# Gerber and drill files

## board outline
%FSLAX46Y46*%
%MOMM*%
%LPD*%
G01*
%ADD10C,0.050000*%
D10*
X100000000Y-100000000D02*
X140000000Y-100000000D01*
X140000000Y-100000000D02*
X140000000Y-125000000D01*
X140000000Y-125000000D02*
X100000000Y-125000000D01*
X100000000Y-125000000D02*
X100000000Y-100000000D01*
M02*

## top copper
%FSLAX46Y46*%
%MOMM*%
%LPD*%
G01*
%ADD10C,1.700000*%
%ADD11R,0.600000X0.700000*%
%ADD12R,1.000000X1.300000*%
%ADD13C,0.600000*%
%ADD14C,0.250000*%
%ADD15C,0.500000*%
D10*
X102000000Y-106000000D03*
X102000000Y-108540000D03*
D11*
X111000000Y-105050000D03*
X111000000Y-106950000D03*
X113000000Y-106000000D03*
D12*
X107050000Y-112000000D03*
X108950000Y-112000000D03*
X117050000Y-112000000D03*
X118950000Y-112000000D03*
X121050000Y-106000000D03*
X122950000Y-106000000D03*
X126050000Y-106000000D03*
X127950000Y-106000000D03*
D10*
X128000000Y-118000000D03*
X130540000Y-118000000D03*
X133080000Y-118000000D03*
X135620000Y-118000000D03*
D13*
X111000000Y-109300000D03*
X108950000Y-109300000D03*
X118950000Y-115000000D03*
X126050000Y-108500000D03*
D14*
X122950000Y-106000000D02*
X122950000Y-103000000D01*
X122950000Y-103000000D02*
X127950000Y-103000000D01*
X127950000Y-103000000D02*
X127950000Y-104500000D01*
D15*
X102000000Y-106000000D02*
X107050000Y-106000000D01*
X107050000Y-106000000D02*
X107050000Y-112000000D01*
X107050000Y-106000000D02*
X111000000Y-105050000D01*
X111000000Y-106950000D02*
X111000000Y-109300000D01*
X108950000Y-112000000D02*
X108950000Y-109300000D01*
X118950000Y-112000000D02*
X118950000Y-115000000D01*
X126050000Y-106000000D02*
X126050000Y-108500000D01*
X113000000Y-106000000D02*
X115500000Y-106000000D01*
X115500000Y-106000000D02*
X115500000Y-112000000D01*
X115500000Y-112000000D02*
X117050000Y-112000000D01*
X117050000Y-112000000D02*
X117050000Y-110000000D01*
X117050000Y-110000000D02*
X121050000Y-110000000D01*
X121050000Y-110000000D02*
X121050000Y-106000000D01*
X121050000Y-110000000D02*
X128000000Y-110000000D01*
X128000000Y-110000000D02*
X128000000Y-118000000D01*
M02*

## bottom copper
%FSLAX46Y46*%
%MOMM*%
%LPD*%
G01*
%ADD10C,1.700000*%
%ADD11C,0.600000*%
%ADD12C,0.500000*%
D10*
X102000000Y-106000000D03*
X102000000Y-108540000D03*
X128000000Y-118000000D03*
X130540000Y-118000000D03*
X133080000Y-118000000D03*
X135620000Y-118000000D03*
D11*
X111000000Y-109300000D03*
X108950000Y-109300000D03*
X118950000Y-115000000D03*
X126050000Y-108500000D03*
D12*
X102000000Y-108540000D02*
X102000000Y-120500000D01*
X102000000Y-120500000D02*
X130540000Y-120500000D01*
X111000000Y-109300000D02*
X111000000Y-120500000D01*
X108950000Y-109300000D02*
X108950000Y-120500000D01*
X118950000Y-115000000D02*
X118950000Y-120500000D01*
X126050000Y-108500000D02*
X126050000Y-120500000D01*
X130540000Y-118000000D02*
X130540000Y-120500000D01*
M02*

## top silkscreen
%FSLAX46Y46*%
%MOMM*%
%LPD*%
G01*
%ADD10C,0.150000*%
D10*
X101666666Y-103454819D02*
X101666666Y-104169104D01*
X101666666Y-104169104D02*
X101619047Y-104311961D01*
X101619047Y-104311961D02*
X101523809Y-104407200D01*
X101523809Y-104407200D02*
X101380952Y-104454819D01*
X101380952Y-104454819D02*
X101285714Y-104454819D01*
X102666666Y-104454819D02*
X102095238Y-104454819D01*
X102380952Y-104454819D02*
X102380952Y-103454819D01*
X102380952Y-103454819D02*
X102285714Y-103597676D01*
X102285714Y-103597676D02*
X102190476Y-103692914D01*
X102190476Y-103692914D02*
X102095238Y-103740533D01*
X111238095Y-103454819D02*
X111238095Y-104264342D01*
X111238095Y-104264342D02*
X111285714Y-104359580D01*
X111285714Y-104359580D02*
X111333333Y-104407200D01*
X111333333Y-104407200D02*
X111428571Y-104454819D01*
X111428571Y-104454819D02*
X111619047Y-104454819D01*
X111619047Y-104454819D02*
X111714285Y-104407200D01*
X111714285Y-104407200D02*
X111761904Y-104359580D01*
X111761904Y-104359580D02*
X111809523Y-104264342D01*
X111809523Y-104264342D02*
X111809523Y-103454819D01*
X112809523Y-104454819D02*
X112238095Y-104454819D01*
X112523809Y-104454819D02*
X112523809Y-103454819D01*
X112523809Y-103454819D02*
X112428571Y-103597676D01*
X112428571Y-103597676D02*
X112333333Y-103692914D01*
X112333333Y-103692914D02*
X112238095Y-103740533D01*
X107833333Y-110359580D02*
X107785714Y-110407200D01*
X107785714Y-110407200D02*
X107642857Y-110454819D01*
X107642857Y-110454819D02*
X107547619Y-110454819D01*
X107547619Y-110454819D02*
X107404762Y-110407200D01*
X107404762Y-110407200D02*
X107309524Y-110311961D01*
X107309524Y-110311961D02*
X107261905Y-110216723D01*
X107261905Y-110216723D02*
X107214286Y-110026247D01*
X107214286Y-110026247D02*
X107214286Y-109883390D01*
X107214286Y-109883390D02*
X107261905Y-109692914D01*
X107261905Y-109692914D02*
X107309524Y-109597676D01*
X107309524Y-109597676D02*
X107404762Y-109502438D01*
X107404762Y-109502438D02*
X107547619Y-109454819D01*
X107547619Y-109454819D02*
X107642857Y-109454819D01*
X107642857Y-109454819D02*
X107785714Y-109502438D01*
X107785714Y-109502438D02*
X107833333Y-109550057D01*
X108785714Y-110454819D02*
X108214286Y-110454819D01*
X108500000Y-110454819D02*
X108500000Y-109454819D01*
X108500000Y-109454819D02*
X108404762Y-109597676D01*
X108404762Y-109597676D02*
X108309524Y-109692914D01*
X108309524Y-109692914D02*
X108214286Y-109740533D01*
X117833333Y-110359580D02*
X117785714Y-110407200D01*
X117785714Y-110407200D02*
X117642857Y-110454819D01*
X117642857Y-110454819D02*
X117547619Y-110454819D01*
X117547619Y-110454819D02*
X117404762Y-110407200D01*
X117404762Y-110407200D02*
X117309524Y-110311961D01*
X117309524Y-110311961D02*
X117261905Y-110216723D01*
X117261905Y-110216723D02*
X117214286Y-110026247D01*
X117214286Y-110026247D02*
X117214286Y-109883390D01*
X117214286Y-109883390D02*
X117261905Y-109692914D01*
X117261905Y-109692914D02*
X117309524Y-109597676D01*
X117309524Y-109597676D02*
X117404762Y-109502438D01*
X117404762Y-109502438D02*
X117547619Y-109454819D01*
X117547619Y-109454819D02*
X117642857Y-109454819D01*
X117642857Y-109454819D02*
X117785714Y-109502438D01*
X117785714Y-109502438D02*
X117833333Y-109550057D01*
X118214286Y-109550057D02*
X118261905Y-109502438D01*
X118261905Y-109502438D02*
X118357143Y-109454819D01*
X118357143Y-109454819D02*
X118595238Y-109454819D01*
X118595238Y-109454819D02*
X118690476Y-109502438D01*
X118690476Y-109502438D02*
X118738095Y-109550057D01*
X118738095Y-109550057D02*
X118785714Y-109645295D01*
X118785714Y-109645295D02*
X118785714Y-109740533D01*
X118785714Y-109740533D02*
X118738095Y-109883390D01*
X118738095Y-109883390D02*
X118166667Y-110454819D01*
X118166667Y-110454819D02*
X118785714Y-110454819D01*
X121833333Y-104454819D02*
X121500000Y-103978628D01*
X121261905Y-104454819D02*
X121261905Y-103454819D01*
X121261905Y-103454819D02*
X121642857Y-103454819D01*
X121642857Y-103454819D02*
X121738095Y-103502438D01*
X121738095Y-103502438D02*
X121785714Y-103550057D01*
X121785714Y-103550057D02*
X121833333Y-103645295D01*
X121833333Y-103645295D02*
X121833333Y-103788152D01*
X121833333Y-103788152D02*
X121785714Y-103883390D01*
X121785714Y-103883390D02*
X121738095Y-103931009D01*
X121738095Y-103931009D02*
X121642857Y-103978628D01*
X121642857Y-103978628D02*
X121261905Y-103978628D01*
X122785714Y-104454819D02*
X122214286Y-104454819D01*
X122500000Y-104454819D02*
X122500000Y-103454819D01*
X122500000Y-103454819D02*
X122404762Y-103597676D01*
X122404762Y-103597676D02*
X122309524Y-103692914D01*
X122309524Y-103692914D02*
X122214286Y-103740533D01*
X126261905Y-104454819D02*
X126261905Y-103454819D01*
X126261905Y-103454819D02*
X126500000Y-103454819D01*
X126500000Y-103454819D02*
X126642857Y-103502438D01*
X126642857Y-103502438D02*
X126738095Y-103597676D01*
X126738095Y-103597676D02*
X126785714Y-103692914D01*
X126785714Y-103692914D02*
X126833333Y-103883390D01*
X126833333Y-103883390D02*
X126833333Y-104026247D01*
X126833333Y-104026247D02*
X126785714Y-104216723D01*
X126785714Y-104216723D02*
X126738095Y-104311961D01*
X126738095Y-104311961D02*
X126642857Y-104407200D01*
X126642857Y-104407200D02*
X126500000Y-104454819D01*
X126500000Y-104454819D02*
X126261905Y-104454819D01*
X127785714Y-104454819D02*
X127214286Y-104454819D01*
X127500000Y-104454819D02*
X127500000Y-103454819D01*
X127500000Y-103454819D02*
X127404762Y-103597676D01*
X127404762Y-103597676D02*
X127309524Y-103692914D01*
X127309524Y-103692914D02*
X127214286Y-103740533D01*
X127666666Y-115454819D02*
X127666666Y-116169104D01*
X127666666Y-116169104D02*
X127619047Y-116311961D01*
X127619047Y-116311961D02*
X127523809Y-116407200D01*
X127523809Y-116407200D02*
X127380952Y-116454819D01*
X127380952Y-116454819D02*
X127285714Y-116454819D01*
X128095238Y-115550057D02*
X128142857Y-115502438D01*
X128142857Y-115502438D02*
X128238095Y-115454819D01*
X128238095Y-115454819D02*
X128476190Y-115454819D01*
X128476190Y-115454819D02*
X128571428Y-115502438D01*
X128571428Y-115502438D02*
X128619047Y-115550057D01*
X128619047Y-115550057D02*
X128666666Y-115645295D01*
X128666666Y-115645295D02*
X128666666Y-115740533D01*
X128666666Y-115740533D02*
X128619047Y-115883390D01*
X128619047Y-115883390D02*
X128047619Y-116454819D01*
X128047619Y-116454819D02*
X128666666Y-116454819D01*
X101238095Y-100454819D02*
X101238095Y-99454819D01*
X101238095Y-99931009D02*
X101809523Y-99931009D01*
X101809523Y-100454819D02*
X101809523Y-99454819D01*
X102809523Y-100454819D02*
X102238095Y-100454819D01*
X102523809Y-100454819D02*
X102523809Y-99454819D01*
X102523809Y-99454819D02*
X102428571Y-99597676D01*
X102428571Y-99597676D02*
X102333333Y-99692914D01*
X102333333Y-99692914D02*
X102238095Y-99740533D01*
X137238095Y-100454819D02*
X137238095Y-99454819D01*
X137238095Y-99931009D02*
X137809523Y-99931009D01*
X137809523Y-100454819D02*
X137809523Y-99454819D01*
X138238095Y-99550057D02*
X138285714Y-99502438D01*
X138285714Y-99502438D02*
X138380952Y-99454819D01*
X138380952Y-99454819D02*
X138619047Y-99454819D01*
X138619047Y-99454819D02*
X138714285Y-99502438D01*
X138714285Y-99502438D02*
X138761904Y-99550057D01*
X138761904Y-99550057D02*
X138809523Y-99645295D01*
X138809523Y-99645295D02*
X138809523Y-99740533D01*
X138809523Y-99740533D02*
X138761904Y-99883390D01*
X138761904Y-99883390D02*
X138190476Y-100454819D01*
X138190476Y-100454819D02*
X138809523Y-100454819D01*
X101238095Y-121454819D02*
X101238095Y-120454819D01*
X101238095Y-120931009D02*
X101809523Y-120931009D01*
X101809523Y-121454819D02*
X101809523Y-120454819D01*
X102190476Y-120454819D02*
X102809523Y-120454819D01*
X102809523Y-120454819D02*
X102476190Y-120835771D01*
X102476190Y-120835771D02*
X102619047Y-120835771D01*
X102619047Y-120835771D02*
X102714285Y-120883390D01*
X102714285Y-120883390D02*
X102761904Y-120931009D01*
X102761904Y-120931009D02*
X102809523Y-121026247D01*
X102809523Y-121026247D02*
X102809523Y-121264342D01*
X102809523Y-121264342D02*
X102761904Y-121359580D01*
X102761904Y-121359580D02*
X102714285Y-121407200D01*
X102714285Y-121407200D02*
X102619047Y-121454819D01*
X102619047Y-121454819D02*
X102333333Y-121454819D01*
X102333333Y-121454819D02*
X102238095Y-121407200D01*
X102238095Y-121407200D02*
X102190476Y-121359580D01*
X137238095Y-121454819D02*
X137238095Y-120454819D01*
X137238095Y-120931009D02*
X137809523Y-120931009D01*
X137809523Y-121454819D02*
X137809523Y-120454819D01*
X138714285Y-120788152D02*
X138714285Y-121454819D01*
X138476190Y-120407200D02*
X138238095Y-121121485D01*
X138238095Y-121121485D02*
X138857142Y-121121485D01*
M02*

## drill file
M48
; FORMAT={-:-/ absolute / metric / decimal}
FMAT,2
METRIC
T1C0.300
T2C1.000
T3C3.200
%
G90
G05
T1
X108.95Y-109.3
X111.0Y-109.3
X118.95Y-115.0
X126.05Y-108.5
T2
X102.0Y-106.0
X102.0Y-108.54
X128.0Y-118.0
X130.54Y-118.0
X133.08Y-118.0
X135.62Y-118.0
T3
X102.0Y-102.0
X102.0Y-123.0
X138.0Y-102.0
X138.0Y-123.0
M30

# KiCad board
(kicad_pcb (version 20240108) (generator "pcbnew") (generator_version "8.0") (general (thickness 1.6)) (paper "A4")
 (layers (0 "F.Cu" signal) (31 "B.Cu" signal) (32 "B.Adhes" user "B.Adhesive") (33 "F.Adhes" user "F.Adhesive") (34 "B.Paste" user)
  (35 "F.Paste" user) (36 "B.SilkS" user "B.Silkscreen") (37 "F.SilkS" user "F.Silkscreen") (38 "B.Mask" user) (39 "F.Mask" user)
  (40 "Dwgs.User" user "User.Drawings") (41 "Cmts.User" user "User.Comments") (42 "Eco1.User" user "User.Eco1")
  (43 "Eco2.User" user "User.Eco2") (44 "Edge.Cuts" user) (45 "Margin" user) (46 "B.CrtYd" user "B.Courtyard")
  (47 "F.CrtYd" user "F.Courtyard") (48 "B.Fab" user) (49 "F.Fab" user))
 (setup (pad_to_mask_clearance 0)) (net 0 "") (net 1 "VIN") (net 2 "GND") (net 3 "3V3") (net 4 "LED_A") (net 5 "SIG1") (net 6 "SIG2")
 (gr_line (start 100 100) (end 140 100) (stroke (width 0.05) (type default)) (layer "Edge.Cuts"))
 (gr_line (start 140 100) (end 140 125) (stroke (width 0.05) (type default)) (layer "Edge.Cuts"))
 (gr_line (start 140 125) (end 100 125) (stroke (width 0.05) (type default)) (layer "Edge.Cuts"))
 (gr_line (start 100 125) (end 100 100) (stroke (width 0.05) (type default)) (layer "Edge.Cuts"))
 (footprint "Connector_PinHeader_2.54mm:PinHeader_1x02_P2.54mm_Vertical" (layer "F.Cu") (at 102 106)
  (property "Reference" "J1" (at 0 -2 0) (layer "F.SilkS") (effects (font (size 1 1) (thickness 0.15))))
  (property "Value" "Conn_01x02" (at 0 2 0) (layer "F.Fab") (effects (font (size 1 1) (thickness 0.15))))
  (pad "1" thru_hole circle (at 0 0) (size 1.7 1.7) (drill 1) (layers "*.Cu" "*.Mask") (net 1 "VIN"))
  (pad "2" thru_hole circle (at 0 2.54) (size 1.7 1.7) (drill 1) (layers "*.Cu" "*.Mask") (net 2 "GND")))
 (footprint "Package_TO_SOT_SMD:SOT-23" (layer "F.Cu") (at 112 106)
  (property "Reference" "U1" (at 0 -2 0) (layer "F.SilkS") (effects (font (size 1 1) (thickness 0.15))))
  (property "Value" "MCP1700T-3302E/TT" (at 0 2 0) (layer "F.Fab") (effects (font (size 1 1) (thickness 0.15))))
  (pad "1" smd rect (at -1 -0.95) (size 0.6 0.7) (layers "F.Cu" "F.Paste" "F.Mask") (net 1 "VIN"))
  (pad "2" smd rect (at -1 0.95) (size 0.6 0.7) (layers "F.Cu" "F.Paste" "F.Mask") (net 2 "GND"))
  (pad "3" smd rect (at 1 0) (size 0.6 0.7) (layers "F.Cu" "F.Paste" "F.Mask") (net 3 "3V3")))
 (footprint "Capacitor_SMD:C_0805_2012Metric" (layer "F.Cu") (at 108 112)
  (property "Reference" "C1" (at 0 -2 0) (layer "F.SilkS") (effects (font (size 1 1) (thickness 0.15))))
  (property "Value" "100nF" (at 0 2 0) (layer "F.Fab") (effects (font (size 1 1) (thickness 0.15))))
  (pad "1" smd rect (at -0.95 0) (size 1 1.3) (layers "F.Cu" "F.Paste" "F.Mask") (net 1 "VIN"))
  (pad "2" smd rect (at 0.95 0) (size 1 1.3) (layers "F.Cu" "F.Paste" "F.Mask") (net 2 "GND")))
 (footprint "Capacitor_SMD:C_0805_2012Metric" (layer "F.Cu") (at 118 112)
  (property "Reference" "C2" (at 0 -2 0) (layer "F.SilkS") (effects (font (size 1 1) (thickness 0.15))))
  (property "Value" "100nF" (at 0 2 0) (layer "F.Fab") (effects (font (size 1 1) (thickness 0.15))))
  (pad "1" smd rect (at -0.95 0) (size 1 1.3) (layers "F.Cu" "F.Paste" "F.Mask") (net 3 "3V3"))
  (pad "2" smd rect (at 0.95 0) (size 1 1.3) (layers "F.Cu" "F.Paste" "F.Mask") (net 2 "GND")))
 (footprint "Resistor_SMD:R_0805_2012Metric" (layer "F.Cu") (at 122 106)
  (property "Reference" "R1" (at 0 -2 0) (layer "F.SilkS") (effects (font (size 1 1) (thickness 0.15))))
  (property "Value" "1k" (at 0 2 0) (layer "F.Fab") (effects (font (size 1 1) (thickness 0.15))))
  (pad "1" smd rect (at -0.95 0) (size 1 1.3) (layers "F.Cu" "F.Paste" "F.Mask") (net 3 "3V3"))
  (pad "2" smd rect (at 0.95 0) (size 1 1.3) (layers "F.Cu" "F.Paste" "F.Mask") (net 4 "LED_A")))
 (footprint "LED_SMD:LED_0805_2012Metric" (layer "F.Cu") (at 127 106)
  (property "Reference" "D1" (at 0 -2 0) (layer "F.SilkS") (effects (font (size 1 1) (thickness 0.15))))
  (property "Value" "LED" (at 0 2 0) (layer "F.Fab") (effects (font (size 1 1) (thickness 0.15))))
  (pad "1" smd rect (at -0.95 0) (size 1 1.3) (layers "F.Cu" "F.Paste" "F.Mask") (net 2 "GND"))
  (pad "2" smd rect (at 0.95 0) (size 1 1.3) (layers "F.Cu" "F.Paste" "F.Mask") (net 4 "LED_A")))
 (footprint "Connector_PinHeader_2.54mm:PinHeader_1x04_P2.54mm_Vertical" (layer "F.Cu") (at 128 118)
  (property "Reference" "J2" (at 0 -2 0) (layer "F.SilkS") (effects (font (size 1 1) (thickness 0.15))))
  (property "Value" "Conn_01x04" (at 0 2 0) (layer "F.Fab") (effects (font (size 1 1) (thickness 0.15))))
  (pad "1" thru_hole circle (at 0 0) (size 1.7 1.7) (drill 1) (layers "*.Cu" "*.Mask") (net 3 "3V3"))
  (pad "2" thru_hole circle (at 2.54 0) (size 1.7 1.7) (drill 1) (layers "*.Cu" "*.Mask") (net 2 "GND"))
  (pad "3" thru_hole circle (at 5.08 0) (size 1.7 1.7) (drill 1) (layers "*.Cu" "*.Mask") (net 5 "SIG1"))
  (pad "4" thru_hole circle (at 7.62 0) (size 1.7 1.7) (drill 1) (layers "*.Cu" "*.Mask") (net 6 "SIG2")))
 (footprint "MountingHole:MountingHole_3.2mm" (layer "F.Cu") (at 102 102)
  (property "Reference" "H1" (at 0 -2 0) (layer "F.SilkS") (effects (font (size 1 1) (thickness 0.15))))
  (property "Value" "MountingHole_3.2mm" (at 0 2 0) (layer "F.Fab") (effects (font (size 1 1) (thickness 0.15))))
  (pad "1" np_thru_hole circle (at 0 0) (size 3.2 3.2) (drill 3.2) (layers "*.Cu" "*.Mask")))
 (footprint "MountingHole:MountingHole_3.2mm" (layer "F.Cu") (at 138 102)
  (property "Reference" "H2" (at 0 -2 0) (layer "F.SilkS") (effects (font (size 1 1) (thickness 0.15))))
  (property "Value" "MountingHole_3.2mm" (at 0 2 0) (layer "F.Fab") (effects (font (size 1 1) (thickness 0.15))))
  (pad "1" np_thru_hole circle (at 0 0) (size 3.2 3.2) (drill 3.2) (layers "*.Cu" "*.Mask")))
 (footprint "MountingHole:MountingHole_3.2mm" (layer "F.Cu") (at 102 123)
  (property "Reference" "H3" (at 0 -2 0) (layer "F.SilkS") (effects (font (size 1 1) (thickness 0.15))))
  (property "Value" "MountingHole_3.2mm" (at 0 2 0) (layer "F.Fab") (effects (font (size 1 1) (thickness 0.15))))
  (pad "1" np_thru_hole circle (at 0 0) (size 3.2 3.2) (drill 3.2) (layers "*.Cu" "*.Mask")))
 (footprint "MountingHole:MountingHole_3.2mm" (layer "F.Cu") (at 138 123)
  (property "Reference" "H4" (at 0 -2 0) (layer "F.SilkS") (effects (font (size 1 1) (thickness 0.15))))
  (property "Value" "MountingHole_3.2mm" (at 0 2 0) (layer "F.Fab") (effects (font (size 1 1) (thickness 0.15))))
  (pad "1" np_thru_hole circle (at 0 0) (size 3.2 3.2) (drill 3.2) (layers "*.Cu" "*.Mask")))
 (segment (start 122.95 106) (end 122.95 103) (width 0.25) (layer "F.Cu") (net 4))
 (segment (start 122.95 103) (end 127.95 103) (width 0.25) (layer "F.Cu") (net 4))
 (segment (start 127.95 103) (end 127.95 104.5) (width 0.25) (layer "F.Cu") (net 4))
 (segment (start 102 106) (end 107.05 106) (width 0.5) (layer "F.Cu") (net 1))
 (segment (start 107.05 106) (end 107.05 112) (width 0.5) (layer "F.Cu") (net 1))
 (segment (start 107.05 106) (end 111 105.05) (width 0.5) (layer "F.Cu") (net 1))
 (segment (start 111 106.95) (end 111 109.3) (width 0.5) (layer "F.Cu") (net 2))
 (segment (start 108.95 112) (end 108.95 109.3) (width 0.5) (layer "F.Cu") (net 2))
 (segment (start 118.95 112) (end 118.95 115) (width 0.5) (layer "F.Cu") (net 2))
 (segment (start 126.05 106) (end 126.05 108.5) (width 0.5) (layer "F.Cu") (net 2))
 (segment (start 113 106) (end 115.5 106) (width 0.5) (layer "F.Cu") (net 3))
 (segment (start 115.5 106) (end 115.5 112) (width 0.5) (layer "F.Cu") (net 3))
 (segment (start 115.5 112) (end 117.05 112) (width 0.5) (layer "F.Cu") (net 3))
 (segment (start 117.05 112) (end 117.05 110) (width 0.5) (layer "F.Cu") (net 3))
 (segment (start 117.05 110) (end 121.05 110) (width 0.5) (layer "F.Cu") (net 3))
 (segment (start 121.05 110) (end 121.05 106) (width 0.5) (layer "F.Cu") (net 3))
 (segment (start 121.05 110) (end 128 110) (width 0.5) (layer "F.Cu") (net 3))
 (segment (start 128 110) (end 128 118) (width 0.5) (layer "F.Cu") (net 3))
 (segment (start 102 108.54) (end 102 120.5) (width 0.5) (layer "B.Cu") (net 2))
 (segment (start 102 120.5) (end 130.54 120.5) (width 0.5) (layer "B.Cu") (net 2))
 (segment (start 111 109.3) (end 111 120.5) (width 0.5) (layer "B.Cu") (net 2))
 (segment (start 108.95 109.3) (end 108.95 120.5) (width 0.5) (layer "B.Cu") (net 2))
 (segment (start 118.95 115) (end 118.95 120.5) (width 0.5) (layer "B.Cu") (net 2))
 (segment (start 126.05 108.5) (end 126.05 120.5) (width 0.5) (layer "B.Cu") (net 2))
 (segment (start 130.54 118) (end 130.54 120.5) (width 0.5) (layer "B.Cu") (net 2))
 (via (at 111 109.3) (size 0.6) (drill 0.3) (layers "F.Cu" "B.Cu") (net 2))
 (via (at 108.95 109.3) (size 0.6) (drill 0.3) (layers "F.Cu" "B.Cu") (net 2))
 (via (at 118.95 115) (size 0.6) (drill 0.3) (layers "F.Cu" "B.Cu") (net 2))
 (via (at 126.05 108.5) (size 0.6) (drill 0.3) (layers "F.Cu" "B.Cu") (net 2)))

